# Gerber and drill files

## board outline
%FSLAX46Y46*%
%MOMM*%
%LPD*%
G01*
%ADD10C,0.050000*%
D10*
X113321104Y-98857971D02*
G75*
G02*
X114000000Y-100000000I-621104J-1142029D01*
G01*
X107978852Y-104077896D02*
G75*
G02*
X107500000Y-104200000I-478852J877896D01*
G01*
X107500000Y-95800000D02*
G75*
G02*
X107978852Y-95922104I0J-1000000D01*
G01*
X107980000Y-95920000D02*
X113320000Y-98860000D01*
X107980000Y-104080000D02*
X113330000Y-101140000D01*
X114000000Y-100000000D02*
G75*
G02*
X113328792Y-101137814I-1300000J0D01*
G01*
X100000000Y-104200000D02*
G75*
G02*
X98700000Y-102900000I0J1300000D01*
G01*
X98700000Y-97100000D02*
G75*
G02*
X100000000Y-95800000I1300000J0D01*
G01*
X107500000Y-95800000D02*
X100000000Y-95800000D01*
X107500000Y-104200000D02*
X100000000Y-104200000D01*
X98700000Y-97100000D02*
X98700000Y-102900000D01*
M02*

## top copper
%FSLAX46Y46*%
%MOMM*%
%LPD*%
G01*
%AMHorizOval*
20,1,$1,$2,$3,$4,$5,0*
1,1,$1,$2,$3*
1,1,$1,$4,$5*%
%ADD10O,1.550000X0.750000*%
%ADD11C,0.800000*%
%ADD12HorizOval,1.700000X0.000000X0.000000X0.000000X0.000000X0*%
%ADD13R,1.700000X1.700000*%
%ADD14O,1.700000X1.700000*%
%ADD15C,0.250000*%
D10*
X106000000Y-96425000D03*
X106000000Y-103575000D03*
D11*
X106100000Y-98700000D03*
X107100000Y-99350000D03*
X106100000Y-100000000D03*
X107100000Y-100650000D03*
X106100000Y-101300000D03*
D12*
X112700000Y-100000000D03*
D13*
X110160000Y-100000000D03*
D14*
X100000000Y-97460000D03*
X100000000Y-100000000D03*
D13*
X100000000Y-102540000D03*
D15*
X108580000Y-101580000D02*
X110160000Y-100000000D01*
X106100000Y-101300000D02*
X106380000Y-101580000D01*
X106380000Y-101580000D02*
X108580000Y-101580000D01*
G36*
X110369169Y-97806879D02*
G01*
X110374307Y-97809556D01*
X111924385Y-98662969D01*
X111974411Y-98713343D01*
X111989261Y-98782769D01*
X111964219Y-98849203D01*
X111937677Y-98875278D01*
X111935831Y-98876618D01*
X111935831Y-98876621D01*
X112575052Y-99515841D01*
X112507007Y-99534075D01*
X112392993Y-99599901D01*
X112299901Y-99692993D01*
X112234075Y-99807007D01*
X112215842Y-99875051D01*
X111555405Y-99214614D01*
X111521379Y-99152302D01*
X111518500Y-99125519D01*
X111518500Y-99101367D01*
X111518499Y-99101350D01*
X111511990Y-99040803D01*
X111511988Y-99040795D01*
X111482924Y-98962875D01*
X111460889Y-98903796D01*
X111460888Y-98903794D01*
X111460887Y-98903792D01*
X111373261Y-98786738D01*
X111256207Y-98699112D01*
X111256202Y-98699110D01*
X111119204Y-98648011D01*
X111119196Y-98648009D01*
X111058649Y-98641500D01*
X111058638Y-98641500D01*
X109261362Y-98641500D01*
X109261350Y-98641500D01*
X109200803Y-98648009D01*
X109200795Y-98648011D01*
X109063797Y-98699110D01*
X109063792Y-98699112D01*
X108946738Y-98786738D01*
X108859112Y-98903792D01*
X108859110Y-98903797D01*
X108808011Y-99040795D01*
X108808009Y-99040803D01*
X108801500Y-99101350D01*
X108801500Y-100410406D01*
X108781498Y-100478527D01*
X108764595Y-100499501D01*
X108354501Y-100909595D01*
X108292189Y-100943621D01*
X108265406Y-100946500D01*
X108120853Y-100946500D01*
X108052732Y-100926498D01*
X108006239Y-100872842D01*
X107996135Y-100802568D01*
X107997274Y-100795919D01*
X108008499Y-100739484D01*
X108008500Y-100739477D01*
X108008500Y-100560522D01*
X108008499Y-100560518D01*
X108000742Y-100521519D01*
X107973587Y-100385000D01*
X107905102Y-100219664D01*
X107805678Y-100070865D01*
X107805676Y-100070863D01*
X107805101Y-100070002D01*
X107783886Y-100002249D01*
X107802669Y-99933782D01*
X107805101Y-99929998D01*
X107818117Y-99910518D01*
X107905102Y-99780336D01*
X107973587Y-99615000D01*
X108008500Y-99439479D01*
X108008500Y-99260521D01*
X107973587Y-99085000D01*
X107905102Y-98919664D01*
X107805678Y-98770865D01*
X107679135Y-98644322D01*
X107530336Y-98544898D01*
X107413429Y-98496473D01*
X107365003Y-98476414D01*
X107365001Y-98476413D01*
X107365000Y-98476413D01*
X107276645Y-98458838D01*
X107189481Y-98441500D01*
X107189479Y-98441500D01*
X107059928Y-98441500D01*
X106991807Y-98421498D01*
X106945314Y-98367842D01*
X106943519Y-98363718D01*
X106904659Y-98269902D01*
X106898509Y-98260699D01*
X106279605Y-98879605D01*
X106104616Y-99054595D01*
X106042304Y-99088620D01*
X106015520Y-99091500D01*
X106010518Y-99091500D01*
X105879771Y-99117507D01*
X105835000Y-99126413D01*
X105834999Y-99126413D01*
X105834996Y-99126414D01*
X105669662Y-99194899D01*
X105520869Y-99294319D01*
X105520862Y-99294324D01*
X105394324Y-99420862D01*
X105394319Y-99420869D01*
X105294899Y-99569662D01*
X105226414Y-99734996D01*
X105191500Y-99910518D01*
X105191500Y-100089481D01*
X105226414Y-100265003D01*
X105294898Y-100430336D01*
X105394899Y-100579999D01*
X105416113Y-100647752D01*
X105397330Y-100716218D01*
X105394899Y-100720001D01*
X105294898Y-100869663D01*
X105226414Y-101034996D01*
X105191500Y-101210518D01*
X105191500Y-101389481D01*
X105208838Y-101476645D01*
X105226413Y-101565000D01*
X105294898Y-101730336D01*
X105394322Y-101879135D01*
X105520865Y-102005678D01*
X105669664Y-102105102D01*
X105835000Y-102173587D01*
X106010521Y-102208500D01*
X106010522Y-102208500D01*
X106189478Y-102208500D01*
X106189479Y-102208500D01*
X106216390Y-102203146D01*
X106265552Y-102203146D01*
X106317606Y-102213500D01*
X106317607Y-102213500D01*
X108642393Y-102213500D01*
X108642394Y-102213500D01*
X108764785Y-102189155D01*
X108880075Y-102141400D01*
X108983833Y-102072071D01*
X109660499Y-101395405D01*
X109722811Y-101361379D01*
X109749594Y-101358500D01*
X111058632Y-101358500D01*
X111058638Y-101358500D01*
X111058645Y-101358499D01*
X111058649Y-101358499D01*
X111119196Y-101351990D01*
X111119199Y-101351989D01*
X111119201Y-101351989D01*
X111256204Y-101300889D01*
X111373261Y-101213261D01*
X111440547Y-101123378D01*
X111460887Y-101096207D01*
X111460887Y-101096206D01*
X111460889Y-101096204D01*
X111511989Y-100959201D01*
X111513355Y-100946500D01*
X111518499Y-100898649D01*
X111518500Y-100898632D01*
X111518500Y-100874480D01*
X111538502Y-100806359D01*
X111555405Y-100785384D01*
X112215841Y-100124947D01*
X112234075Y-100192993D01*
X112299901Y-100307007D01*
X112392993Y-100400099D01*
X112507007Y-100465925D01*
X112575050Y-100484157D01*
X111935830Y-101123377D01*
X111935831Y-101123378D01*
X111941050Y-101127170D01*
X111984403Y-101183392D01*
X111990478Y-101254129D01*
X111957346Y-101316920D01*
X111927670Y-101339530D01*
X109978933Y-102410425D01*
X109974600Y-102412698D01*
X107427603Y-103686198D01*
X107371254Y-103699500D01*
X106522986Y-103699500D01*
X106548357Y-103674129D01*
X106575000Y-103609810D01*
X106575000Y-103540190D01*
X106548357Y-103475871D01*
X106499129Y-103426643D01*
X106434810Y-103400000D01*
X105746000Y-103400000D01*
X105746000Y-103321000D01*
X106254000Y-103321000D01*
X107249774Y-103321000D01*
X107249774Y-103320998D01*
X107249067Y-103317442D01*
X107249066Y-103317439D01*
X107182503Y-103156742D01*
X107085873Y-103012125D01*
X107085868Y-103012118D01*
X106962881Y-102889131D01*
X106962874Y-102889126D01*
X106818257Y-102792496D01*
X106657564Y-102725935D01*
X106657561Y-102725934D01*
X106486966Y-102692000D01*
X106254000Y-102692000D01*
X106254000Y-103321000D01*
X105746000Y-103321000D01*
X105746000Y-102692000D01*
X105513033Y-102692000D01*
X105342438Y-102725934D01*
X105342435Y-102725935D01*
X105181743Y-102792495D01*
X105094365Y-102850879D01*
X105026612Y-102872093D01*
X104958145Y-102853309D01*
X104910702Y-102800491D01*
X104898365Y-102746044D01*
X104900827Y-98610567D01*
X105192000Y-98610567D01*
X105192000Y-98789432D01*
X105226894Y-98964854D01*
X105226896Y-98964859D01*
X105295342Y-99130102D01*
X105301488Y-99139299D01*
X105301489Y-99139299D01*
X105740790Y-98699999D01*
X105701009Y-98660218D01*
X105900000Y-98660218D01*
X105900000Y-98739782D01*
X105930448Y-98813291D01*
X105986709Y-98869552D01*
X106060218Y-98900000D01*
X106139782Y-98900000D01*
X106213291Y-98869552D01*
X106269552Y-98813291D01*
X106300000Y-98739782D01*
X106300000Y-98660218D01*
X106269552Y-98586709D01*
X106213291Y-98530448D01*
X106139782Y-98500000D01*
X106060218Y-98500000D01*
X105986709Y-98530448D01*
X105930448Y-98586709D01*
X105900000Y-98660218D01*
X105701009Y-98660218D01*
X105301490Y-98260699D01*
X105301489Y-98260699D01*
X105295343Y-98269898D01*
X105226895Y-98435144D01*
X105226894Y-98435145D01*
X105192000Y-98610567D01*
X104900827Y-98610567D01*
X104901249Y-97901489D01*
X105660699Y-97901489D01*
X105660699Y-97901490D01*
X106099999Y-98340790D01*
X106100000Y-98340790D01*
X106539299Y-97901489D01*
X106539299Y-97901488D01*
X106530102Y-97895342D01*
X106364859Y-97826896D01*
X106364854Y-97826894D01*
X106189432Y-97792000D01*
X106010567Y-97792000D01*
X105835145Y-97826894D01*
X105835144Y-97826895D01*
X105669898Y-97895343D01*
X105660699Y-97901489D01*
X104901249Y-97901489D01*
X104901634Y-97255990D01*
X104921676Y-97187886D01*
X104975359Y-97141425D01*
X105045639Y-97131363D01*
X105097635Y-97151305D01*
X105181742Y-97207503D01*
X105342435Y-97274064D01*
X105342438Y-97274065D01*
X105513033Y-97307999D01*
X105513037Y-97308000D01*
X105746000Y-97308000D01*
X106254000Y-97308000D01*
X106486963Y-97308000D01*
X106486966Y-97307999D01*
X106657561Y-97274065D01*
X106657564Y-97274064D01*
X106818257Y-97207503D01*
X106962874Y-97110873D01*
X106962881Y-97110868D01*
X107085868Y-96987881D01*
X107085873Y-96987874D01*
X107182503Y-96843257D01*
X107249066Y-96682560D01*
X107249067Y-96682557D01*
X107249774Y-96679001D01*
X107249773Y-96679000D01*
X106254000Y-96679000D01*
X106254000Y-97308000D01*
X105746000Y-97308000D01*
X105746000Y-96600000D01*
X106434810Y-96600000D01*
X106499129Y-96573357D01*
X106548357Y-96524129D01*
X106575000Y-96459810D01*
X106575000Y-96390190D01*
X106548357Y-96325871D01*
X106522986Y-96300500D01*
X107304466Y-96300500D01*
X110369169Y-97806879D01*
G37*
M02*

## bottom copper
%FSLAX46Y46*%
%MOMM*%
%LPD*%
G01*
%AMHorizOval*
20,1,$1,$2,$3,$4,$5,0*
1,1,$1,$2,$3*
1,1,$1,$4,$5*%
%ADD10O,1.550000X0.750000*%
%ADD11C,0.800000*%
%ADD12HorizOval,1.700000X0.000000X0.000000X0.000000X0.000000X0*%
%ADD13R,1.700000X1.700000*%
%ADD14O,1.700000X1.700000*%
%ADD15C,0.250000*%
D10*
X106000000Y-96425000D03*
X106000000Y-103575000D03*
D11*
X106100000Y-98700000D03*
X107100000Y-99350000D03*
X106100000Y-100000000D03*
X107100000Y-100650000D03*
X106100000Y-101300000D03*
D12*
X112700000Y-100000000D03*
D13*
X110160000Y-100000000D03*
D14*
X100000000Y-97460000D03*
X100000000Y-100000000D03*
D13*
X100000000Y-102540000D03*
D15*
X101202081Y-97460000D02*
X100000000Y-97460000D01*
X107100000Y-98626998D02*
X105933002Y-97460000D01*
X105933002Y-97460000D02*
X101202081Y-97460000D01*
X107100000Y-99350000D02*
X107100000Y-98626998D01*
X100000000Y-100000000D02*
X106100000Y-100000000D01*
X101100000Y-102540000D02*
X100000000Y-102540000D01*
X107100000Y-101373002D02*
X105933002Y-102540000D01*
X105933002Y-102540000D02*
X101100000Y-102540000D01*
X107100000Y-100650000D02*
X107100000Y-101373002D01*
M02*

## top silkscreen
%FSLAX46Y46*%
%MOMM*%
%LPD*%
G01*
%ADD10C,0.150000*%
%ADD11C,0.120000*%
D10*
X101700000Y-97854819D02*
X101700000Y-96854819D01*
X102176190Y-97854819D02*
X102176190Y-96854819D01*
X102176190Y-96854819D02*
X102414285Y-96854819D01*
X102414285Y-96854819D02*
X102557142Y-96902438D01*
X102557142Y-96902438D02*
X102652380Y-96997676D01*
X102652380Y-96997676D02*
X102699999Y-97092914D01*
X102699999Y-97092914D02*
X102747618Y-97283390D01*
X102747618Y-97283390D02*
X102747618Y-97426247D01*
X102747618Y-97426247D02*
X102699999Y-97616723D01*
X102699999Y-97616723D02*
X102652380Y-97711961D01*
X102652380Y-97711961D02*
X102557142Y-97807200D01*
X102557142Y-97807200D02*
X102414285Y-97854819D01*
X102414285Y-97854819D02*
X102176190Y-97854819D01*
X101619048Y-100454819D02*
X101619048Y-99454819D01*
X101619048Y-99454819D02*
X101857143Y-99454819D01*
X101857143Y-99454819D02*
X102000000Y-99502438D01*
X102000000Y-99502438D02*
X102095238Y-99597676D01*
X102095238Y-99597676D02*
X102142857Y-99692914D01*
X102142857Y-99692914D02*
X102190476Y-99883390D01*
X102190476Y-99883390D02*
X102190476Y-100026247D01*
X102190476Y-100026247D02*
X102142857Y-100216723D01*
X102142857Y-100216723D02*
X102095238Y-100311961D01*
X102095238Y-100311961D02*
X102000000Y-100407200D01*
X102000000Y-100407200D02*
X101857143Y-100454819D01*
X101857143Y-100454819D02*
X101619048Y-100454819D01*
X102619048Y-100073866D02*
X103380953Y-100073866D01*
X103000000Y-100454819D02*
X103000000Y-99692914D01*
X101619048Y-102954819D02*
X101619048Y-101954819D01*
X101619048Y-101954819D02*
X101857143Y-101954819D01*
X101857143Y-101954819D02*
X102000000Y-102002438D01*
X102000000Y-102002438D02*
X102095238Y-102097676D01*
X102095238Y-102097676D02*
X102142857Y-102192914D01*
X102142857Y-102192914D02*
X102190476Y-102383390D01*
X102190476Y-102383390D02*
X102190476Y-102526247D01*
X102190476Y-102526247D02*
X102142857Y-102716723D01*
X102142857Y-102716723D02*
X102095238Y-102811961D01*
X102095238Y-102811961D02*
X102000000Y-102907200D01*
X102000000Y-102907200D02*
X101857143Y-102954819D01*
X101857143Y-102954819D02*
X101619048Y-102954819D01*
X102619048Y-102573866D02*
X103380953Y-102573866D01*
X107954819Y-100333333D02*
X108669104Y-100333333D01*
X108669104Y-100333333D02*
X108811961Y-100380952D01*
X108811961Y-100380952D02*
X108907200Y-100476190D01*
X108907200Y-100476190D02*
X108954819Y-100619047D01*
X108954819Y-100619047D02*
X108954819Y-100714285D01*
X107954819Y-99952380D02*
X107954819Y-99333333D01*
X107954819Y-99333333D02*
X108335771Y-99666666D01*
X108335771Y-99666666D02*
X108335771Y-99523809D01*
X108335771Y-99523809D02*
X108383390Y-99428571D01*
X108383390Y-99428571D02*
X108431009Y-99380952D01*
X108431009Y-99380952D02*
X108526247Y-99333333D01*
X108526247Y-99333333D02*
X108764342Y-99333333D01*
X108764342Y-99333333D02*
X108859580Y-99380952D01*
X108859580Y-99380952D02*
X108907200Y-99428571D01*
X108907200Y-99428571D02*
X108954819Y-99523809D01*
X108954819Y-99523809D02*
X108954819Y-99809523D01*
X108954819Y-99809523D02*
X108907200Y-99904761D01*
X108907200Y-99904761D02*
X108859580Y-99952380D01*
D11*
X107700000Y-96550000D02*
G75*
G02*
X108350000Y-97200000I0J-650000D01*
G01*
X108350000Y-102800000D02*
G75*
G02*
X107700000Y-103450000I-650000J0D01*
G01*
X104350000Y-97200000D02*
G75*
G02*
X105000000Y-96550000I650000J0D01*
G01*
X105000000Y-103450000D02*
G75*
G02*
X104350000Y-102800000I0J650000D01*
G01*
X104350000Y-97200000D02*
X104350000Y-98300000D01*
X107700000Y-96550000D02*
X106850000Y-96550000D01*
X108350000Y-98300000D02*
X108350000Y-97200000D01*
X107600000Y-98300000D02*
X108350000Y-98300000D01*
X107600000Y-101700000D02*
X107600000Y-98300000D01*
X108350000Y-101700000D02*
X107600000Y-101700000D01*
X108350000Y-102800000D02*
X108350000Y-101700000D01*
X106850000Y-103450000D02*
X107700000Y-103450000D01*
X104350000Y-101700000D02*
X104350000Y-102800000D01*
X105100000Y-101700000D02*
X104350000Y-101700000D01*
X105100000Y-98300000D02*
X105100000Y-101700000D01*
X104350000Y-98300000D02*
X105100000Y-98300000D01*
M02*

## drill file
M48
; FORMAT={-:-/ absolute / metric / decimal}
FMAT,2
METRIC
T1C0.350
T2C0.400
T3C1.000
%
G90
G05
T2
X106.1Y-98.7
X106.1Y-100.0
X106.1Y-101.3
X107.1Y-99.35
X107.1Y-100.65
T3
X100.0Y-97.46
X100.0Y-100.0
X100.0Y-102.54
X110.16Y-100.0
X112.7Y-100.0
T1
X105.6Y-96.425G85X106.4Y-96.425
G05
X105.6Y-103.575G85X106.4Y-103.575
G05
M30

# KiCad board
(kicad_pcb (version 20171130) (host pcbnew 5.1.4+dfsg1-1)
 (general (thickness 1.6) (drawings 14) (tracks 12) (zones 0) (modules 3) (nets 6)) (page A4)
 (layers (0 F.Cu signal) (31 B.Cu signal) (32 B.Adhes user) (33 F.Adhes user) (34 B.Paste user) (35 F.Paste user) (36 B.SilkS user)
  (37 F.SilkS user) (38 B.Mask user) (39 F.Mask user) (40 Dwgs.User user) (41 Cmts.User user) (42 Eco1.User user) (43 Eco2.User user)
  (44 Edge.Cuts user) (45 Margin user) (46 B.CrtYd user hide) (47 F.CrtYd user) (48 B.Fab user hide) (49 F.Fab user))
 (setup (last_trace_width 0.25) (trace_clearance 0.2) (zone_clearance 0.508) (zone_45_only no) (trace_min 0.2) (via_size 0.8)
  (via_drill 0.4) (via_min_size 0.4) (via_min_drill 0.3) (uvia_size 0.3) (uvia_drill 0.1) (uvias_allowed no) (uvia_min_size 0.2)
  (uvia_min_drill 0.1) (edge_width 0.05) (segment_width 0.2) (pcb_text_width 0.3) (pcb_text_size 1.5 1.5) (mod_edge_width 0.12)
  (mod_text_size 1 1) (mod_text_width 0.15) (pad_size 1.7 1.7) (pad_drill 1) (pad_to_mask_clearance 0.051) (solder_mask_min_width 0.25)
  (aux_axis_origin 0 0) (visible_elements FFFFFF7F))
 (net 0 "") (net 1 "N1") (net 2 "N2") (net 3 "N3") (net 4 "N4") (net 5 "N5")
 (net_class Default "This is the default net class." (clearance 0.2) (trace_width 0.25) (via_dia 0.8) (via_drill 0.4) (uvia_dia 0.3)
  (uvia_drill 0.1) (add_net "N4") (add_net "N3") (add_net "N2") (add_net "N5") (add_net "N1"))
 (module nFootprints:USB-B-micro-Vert (layer F.Cu) (at 106.35 100 90)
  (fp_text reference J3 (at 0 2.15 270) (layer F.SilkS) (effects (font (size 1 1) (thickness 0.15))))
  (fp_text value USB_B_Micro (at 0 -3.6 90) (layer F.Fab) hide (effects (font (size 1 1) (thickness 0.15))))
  (fp_arc (start 2.8 1.35) (end 2.8 2) (angle -90) (layer F.SilkS) (width 0.12))
  (fp_arc (start -2.8 1.35) (end -2.8 2) (angle 90) (layer F.SilkS) (width 0.12))
  (fp_arc (start 2.8 -1.35) (end 3.45 -1.35) (angle -90) (layer F.SilkS) (width 0.12))
  (fp_arc (start -2.8 -1.35) (end -2.8 -2) (angle -90) (layer F.SilkS) (width 0.12))
  (fp_line (start 2.8 -2) (end 1.7 -2) (layer F.SilkS) (width 0.12))
  (fp_line (start 3.45 1.35) (end 3.45 0.5) (layer F.SilkS) (width 0.12))
  (fp_line (start 1.7 2) (end 2.8 2) (layer F.SilkS) (width 0.12))
  (fp_line (start 1.7 1.25) (end 1.7 2) (layer F.SilkS) (width 0.12))
  (fp_line (start -1.7 1.25) (end 1.7 1.25) (layer F.SilkS) (width 0.12))
  (fp_line (start -1.7 2) (end -1.7 1.25) (layer F.SilkS) (width 0.12))
  (fp_line (start -2.8 2) (end -1.7 2) (layer F.SilkS) (width 0.12))
  (fp_line (start -3.45 0.5) (end -3.45 1.35) (layer F.SilkS) (width 0.12))
  (fp_line (start -1.7 -2) (end -2.8 -2) (layer F.SilkS) (width 0.12))
  (fp_line (start -1.7 -1.25) (end -1.7 -2) (layer F.SilkS) (width 0.12))
  (fp_line (start 1.7 -1.25) (end -1.7 -1.25) (layer F.SilkS) (width 0.12))
  (fp_line (start 1.7 -2) (end 1.7 -1.25) (layer F.SilkS) (width 0.12))
  (pad 6 thru_hole oval (at 3.575 -0.35 90) (size 0.75 1.55) (drill oval 0.35 1.15) (layers *.Cu *.Mask) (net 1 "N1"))
  (pad 6 thru_hole oval (at -3.575 -0.35 90) (size 0.75 1.55) (drill oval 0.35 1.15) (layers *.Cu *.Mask) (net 1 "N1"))
  (pad 5 thru_hole circle (at 1.3 -0.25 90) (size 0.8 0.8) (drill 0.4) (layers *.Cu *.Mask) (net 1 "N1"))
  (pad 4 thru_hole circle (at 0.65 0.75 90) (size 0.8 0.8) (drill 0.4) (layers *.Cu *.Mask) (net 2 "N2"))
  (pad 3 thru_hole circle (at 0 -0.25 90) (size 0.8 0.8) (drill 0.4) (layers *.Cu *.Mask) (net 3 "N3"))
  (pad 2 thru_hole circle (at -0.65 0.75 90) (size 0.8 0.8) (drill 0.4) (layers *.Cu *.Mask) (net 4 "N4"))
  (pad 1 thru_hole circle (at -1.3 -0.25 90) (size 0.8 0.8) (drill 0.4) (layers *.Cu *.Mask) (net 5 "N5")))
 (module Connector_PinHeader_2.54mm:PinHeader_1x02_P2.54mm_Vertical (layer B.Cu) (at 110.16 100 270)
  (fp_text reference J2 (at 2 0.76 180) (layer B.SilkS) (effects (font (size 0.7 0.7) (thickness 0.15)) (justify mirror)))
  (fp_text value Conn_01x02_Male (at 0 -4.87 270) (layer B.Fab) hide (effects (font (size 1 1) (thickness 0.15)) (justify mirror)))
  (pad 2 thru_hole oval (at 0 -2.54 225) (size 1.7 1.7) (drill 1) (layers *.Cu *.Mask) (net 1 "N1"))
  (pad 1 thru_hole rect (at 0 0 270) (size 1.7 1.7) (drill 1) (layers *.Cu *.Mask) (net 5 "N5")))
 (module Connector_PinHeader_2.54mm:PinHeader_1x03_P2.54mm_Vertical (layer B.Cu) (at 100 102.54)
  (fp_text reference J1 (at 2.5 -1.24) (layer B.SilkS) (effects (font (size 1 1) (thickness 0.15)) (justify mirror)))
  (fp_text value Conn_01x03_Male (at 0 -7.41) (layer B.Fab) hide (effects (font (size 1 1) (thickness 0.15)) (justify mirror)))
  (pad 3 thru_hole oval (at 0 -5.08) (size 1.7 1.7) (drill 1) (layers *.Cu *.Mask) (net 2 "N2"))
  (pad 2 thru_hole oval (at 0 -2.54) (size 1.7 1.7) (drill 1) (layers *.Cu *.Mask) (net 3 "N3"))
  (pad 1 thru_hole rect (at 0 0) (size 1.7 1.7) (drill 1) (layers *.Cu *.Mask) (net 4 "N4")))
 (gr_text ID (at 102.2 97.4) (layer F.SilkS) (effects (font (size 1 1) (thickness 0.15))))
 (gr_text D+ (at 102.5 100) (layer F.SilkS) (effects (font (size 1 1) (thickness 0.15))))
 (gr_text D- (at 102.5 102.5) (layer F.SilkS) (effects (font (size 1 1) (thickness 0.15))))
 (gr_arc (start 112.7 100) (end 114 100) (angle -61.46001481) (layer Edge.Cuts) (width 0.05))
 (gr_arc (start 107.5 103.2) (end 107.5 104.2) (angle -28.61045967) (layer Edge.Cuts) (width 0.05))
 (gr_arc (start 107.5 96.8) (end 107.5 95.8) (angle 28.61045967) (layer Edge.Cuts) (width 0.05))
 (gr_line (start 107.98 95.92) (end 113.32 98.86) (layer Edge.Cuts) (width 0.05))
 (gr_line (start 107.98 104.08) (end 113.33 101.14) (layer Edge.Cuts) (width 0.05))
 (gr_arc (start 112.7 100) (end 114 100) (angle 61.07357416) (layer Edge.Cuts) (width 0.05))
 (gr_arc (start 100 102.9) (end 98.7 102.9) (angle -90) (layer Edge.Cuts) (width 0.05))
 (gr_arc (start 100 97.1) (end 100 95.8) (angle -90) (layer Edge.Cuts) (width 0.05))
 (gr_line (start 107.5 95.8) (end 100 95.8) (layer Edge.Cuts) (width 0.05))
 (gr_line (start 107.5 104.2) (end 100 104.2) (layer Edge.Cuts) (width 0.05))
 (gr_line (start 98.7 97.1) (end 98.7 102.9) (layer Edge.Cuts) (width 0.05))
 (segment (start 101.202081 97.46) (end 100 97.46) (width 0.25) (layer B.Cu) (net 2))
 (segment (start 107.1 98.626998) (end 105.933002 97.46) (width 0.25) (layer B.Cu) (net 2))
 (segment (start 105.933002 97.46) (end 101.202081 97.46) (width 0.25) (layer B.Cu) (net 2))
 (segment (start 107.1 99.35) (end 107.1 98.626998) (width 0.25) (layer B.Cu) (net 2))
 (segment (start 100 100) (end 106.1 100) (width 0.25) (layer B.Cu) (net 3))
 (segment (start 101.1 102.54) (end 100 102.54) (width 0.25) (layer B.Cu) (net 4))
 (segment (start 107.1 101.373002) (end 105.933002 102.54) (width 0.25) (layer B.Cu) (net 4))
 (segment (start 105.933002 102.54) (end 101.1 102.54) (width 0.25) (layer B.Cu) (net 4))
 (segment (start 107.1 100.65) (end 107.1 101.373002) (width 0.25) (layer B.Cu) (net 4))
 (segment (start 108.58 101.58) (end 110.16 100) (width 0.25) (layer F.Cu) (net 5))
 (segment (start 106.1 101.3) (end 106.38 101.58) (width 0.25) (layer F.Cu) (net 5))
 (segment (start 106.38 101.58) (end 108.58 101.58) (width 0.25) (layer F.Cu) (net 5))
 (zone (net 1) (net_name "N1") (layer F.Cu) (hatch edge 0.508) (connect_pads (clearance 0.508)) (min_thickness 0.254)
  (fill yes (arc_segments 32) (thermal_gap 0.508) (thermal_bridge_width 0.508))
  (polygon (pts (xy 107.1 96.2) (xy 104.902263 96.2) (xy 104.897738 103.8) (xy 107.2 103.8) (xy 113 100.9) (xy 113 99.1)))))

